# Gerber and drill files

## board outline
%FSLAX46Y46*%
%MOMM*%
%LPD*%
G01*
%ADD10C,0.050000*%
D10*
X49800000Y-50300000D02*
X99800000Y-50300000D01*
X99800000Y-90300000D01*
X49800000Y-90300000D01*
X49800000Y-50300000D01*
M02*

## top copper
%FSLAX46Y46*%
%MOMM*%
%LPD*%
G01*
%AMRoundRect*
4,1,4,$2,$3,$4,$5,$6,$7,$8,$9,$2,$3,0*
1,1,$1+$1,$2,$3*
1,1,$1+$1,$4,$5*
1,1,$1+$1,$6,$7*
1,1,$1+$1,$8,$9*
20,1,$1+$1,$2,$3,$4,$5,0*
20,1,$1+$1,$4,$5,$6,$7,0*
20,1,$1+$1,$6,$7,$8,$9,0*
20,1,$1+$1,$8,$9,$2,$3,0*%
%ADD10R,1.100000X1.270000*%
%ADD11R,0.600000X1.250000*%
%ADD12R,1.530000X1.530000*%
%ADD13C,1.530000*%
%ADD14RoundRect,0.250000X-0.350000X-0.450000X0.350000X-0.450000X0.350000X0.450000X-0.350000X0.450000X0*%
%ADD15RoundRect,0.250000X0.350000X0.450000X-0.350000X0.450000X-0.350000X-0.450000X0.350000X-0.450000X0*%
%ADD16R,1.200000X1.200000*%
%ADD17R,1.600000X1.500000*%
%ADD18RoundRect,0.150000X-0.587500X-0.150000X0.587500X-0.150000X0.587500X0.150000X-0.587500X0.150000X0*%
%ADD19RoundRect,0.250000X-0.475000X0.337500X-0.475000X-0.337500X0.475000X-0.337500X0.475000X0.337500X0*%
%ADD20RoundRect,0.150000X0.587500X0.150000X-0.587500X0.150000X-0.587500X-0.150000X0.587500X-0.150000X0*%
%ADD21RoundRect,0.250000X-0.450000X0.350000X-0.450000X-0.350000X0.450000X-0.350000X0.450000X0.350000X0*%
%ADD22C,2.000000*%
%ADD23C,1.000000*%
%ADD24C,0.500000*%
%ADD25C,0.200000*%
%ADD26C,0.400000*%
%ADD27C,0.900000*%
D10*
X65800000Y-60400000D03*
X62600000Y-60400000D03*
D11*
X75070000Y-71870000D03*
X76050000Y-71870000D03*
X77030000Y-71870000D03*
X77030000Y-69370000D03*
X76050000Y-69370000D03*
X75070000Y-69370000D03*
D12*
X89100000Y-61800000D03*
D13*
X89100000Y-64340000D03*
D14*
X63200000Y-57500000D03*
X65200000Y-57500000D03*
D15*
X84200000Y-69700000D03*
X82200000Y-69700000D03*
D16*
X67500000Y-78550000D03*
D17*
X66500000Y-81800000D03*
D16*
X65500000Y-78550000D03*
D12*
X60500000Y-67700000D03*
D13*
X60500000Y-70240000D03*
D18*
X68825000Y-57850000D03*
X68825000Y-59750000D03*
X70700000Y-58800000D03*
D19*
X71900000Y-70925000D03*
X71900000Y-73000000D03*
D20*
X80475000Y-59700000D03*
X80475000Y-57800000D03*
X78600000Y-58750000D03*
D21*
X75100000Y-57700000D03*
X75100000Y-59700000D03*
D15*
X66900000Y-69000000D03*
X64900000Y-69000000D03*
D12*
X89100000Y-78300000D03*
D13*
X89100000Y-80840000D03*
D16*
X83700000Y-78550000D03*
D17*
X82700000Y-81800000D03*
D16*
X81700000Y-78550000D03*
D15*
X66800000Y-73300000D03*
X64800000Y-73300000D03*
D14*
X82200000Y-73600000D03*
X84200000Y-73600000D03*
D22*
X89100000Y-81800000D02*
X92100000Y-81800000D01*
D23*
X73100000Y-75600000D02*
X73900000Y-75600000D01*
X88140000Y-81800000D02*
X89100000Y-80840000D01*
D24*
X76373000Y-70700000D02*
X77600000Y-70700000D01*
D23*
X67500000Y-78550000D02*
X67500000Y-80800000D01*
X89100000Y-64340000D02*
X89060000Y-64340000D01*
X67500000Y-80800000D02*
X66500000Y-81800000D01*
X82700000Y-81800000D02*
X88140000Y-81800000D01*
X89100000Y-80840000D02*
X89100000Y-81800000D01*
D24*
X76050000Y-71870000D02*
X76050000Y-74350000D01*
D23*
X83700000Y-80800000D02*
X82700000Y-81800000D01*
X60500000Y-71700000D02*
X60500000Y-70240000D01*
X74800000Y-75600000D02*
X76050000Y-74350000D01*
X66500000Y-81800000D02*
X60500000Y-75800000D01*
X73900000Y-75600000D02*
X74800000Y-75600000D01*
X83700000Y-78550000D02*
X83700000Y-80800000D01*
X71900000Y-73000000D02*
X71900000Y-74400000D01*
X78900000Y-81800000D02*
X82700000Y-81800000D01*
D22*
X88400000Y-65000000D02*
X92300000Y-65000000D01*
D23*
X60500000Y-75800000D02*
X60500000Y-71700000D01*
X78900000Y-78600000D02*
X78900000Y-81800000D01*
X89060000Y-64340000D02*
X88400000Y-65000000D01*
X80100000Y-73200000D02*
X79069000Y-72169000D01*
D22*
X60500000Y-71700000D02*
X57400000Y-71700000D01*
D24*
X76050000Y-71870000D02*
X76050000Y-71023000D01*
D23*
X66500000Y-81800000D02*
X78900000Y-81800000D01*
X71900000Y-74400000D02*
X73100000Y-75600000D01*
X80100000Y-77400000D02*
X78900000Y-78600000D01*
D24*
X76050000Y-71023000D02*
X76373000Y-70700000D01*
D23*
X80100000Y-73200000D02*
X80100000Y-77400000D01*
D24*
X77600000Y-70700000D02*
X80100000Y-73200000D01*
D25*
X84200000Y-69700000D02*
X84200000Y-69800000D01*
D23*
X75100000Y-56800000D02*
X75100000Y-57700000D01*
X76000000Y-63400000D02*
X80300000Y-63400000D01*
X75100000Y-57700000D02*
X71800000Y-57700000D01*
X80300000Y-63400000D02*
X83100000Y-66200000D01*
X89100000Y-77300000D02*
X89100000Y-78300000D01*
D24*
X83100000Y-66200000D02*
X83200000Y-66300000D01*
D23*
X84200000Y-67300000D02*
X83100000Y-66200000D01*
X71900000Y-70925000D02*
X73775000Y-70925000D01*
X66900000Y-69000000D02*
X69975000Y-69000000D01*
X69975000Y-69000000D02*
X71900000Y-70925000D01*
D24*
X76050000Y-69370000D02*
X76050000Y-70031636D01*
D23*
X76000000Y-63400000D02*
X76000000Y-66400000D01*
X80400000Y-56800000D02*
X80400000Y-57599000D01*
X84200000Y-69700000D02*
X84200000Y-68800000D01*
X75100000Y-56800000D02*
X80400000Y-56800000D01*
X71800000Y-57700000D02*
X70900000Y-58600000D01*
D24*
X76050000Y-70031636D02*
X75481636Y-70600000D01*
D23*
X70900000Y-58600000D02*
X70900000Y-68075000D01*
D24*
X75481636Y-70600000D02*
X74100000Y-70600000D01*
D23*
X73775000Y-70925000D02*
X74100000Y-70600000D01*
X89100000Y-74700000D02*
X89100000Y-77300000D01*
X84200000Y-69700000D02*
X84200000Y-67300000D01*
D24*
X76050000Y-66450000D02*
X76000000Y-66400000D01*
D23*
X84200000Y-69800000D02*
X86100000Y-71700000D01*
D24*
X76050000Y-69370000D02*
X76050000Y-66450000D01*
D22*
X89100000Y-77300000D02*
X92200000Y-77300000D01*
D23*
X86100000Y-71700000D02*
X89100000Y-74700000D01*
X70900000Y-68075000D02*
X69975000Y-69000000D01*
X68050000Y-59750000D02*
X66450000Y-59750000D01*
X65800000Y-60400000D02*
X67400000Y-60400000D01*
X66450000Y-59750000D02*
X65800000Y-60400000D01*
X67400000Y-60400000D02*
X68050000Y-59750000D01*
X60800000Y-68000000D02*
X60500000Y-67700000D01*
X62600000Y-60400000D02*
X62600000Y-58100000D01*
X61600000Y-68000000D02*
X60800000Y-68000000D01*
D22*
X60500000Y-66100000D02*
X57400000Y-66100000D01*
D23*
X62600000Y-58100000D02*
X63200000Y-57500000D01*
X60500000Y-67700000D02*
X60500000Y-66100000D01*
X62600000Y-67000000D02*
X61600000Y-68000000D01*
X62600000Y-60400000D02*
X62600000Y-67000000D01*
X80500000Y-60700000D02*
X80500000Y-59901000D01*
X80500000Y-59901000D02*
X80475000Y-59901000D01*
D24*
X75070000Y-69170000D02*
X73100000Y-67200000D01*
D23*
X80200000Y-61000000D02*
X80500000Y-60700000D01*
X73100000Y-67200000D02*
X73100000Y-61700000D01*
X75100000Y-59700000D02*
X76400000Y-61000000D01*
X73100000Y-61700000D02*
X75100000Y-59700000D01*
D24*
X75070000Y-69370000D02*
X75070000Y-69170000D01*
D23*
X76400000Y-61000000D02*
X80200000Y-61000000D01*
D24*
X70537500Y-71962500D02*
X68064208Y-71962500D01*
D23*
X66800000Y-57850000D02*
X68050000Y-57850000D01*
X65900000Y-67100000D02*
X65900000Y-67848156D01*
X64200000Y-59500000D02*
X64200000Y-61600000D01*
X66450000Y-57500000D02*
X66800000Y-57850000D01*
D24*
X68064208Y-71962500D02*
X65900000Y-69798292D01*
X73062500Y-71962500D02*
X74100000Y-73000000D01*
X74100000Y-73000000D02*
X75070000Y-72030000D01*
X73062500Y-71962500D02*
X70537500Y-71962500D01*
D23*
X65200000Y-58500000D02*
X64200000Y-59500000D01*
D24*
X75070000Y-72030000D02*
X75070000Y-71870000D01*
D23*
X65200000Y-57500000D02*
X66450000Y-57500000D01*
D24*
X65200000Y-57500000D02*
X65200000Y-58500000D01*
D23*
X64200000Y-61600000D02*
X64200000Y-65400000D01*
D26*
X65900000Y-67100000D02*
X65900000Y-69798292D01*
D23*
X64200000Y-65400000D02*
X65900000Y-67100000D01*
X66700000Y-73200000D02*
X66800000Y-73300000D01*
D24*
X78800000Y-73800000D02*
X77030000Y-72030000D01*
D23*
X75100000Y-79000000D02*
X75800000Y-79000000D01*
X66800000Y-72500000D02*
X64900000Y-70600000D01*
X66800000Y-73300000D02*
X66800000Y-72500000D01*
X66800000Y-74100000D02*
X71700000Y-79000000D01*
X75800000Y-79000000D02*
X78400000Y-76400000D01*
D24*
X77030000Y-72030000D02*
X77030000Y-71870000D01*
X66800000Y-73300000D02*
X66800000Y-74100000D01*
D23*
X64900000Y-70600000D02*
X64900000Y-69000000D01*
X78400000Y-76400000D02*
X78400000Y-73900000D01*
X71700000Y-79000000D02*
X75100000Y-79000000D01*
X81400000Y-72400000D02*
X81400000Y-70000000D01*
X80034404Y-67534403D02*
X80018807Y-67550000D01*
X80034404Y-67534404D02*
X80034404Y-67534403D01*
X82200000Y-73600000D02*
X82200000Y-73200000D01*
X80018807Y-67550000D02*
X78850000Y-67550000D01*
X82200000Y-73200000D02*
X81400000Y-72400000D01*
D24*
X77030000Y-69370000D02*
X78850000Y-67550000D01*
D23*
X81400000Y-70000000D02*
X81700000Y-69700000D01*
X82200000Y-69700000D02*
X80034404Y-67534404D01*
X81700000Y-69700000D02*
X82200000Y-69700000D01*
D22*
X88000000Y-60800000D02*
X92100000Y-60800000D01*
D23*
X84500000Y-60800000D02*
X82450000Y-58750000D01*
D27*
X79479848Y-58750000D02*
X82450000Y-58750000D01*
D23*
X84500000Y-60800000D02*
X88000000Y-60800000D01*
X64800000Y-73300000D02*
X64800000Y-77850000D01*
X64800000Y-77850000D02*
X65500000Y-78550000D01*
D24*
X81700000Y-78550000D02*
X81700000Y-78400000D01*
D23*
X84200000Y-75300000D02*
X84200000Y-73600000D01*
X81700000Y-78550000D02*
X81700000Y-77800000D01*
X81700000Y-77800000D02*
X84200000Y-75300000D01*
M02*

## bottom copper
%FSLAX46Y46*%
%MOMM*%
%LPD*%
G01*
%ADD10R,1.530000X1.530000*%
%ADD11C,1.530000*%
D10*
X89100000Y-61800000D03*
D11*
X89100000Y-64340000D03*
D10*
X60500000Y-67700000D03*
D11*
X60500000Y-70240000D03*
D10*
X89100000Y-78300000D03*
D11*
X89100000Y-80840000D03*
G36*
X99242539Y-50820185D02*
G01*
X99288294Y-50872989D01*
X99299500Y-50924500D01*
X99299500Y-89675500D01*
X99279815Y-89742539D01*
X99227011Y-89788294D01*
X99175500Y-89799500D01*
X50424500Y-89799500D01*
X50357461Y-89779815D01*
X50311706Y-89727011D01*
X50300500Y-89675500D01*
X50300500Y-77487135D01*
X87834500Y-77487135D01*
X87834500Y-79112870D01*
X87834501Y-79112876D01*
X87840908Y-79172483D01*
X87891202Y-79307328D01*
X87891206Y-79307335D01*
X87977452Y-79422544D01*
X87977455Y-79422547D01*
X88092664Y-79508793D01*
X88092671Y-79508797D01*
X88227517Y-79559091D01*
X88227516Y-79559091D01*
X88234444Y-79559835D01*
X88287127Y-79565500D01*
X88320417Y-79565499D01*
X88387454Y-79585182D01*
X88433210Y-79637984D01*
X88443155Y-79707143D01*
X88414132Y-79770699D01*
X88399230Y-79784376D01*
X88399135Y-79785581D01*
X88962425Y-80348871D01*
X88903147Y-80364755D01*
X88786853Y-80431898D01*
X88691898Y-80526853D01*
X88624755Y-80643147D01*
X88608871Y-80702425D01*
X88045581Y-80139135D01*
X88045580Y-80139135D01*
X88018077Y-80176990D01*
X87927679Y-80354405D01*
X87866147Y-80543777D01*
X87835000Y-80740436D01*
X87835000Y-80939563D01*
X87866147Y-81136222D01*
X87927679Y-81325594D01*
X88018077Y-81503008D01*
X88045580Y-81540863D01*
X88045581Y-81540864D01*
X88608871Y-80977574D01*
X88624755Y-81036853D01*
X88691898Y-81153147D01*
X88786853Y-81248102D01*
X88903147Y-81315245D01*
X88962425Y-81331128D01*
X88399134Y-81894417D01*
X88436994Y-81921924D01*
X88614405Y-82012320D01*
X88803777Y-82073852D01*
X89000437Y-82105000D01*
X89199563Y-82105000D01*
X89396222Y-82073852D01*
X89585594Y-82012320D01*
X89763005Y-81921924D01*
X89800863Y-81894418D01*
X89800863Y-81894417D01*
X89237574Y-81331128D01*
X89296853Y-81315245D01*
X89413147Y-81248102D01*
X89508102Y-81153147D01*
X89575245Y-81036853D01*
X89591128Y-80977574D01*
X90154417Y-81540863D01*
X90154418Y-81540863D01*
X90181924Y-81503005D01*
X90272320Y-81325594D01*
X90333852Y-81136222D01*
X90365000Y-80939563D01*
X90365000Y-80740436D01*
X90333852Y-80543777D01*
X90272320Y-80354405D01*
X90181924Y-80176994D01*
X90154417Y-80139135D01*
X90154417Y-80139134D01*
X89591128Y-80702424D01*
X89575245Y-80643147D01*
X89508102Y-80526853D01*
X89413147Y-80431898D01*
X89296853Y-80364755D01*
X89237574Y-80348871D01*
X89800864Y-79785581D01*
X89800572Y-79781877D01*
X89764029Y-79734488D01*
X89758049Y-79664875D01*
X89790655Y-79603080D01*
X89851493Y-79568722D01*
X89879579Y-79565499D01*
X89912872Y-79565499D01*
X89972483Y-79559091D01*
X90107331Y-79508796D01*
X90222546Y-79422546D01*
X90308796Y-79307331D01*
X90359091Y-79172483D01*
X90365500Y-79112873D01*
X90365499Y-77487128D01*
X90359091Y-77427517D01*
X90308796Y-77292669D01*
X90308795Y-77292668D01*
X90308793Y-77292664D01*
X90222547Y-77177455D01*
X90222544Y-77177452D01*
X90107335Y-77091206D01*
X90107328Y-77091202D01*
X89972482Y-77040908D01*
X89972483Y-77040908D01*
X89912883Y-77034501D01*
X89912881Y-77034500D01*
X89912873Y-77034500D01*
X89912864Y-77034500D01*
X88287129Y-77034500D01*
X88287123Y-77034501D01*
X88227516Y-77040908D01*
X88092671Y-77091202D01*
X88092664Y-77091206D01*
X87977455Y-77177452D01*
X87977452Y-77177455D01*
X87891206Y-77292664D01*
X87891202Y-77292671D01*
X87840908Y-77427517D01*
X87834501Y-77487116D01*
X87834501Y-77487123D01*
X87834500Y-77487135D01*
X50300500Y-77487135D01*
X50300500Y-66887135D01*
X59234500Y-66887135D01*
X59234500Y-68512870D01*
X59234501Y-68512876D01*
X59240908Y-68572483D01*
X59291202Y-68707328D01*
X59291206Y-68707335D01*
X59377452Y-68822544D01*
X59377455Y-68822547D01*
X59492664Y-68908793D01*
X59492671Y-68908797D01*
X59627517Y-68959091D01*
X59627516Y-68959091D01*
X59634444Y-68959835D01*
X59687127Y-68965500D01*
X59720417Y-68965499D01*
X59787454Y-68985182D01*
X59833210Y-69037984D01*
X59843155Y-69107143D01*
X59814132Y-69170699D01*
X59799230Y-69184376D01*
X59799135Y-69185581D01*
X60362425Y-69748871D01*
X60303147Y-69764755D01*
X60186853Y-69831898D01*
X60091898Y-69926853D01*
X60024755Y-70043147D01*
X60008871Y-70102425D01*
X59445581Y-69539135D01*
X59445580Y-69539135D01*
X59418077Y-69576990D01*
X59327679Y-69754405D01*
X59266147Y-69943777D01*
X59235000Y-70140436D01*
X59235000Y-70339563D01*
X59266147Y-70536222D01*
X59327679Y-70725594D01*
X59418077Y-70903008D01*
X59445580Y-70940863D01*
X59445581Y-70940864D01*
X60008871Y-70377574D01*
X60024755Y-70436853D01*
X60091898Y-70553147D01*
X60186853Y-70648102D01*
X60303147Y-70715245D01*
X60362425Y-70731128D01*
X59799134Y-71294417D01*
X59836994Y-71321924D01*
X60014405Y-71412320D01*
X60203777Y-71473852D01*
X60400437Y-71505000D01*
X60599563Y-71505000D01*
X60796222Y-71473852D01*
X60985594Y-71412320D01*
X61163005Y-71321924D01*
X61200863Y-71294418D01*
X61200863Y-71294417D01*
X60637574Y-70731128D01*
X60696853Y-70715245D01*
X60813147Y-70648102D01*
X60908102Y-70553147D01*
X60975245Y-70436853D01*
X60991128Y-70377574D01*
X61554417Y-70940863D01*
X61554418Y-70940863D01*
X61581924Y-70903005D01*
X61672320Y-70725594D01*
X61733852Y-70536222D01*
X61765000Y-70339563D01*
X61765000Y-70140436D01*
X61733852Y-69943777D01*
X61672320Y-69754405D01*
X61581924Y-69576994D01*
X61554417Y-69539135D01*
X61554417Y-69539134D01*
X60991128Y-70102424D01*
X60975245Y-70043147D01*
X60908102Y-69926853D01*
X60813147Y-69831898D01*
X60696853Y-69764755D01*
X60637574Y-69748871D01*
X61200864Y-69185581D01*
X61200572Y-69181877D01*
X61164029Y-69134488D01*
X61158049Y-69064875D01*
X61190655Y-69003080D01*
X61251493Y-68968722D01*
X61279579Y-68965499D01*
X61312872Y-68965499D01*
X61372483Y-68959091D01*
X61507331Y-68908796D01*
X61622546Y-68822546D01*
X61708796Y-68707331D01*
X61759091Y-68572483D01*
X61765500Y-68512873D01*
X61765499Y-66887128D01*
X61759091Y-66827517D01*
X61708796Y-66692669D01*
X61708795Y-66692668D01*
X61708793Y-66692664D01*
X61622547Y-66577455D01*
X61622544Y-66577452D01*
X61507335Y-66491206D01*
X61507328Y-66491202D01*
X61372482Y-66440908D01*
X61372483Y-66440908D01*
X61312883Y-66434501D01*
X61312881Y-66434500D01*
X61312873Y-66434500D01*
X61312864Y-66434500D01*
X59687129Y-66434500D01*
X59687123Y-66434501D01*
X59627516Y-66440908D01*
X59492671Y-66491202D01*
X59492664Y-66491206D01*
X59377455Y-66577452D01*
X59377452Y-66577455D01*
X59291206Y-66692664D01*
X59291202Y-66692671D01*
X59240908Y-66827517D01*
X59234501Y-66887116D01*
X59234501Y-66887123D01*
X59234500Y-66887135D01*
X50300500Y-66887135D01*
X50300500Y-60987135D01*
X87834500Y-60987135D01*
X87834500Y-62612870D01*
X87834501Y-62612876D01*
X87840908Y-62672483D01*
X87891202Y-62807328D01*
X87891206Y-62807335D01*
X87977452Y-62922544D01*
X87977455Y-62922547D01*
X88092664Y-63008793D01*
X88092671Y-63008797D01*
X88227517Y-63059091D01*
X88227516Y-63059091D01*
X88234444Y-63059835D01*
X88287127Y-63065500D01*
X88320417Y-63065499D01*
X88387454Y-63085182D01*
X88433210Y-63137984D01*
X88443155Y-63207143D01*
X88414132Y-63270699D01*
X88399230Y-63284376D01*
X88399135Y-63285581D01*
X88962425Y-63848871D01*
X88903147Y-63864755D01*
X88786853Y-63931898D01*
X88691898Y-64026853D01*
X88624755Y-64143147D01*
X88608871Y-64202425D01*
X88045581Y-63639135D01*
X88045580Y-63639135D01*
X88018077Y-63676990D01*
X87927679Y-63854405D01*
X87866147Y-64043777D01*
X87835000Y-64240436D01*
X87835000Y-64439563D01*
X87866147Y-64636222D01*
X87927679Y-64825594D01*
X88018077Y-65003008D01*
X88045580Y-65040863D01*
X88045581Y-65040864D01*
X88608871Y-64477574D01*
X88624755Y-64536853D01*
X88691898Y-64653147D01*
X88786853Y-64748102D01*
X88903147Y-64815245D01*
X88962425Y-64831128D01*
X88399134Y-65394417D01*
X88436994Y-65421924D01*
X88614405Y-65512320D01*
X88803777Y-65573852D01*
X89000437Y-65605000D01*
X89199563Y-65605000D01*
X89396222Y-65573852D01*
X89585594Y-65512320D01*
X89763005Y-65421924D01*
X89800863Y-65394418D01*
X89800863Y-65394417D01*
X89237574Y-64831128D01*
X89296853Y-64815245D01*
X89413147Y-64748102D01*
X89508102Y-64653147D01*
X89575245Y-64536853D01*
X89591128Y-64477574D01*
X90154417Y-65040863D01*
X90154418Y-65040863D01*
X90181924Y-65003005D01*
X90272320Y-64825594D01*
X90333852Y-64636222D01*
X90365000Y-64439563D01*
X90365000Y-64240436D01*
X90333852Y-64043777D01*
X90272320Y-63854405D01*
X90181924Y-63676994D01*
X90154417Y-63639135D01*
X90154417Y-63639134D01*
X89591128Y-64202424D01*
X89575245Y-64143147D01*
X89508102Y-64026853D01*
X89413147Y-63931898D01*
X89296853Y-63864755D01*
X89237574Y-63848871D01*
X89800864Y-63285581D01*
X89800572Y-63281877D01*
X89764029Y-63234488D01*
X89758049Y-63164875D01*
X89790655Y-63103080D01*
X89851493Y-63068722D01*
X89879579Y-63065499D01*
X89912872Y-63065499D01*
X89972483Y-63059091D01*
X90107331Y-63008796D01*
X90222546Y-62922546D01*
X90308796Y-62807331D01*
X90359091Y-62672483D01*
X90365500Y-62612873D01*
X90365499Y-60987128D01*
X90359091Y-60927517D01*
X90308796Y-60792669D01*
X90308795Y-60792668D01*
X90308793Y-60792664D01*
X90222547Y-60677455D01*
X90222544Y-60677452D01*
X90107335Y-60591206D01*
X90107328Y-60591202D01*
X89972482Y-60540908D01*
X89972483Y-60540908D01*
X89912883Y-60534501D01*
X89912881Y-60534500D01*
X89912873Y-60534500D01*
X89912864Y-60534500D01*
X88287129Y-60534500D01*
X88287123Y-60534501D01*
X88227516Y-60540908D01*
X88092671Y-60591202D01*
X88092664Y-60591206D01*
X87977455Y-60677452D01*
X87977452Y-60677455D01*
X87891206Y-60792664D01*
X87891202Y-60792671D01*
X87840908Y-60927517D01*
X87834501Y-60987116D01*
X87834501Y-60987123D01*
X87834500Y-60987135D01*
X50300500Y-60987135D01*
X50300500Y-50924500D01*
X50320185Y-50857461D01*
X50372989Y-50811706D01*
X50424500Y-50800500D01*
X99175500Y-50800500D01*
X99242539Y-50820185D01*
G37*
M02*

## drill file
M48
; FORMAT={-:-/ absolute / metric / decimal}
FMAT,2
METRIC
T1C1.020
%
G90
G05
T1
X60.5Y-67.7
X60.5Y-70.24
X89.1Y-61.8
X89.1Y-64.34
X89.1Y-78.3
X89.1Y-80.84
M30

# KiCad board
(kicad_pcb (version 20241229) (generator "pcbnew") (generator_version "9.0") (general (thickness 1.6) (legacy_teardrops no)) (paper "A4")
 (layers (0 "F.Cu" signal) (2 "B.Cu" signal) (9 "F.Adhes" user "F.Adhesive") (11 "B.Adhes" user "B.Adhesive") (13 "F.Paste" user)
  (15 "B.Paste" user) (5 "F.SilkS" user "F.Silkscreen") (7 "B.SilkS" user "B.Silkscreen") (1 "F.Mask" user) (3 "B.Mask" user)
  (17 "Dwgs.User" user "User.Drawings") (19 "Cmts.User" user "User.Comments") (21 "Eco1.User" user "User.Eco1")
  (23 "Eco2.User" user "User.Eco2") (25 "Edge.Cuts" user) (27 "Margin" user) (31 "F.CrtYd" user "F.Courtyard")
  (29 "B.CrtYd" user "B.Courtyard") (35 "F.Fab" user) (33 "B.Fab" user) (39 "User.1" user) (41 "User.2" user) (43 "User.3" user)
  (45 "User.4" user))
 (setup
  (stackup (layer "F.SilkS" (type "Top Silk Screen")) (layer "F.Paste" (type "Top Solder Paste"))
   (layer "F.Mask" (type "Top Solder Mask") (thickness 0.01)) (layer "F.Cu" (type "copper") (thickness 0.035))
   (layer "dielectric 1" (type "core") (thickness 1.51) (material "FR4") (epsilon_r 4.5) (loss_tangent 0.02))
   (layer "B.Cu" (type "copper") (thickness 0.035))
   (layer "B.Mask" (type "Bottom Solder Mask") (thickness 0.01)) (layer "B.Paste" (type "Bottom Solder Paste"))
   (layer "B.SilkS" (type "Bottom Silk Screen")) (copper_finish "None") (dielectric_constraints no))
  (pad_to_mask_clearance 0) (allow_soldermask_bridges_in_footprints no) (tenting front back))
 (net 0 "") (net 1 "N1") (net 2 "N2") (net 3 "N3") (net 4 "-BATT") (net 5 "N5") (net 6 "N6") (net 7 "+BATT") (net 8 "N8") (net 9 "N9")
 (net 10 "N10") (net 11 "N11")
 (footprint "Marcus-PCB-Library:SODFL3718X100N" (layer "F.Cu") (at 64.2 60.4 180)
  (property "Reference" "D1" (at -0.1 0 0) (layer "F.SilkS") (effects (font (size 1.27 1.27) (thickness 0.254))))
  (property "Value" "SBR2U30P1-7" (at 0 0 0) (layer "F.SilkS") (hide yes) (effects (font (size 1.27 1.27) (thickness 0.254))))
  (pad "1" smd rect (at -1.6 0 180) (size 1.1 1.27) (layers "F.Cu" "F.Mask" "F.Paste") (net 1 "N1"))
  (pad "2" smd rect (at 1.6 0 180) (size 1.1 1.27) (layers "F.Cu" "F.Mask" "F.Paste") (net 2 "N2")))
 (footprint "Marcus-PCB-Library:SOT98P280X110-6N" (layer "F.Cu") (at 76.05 70.62 90)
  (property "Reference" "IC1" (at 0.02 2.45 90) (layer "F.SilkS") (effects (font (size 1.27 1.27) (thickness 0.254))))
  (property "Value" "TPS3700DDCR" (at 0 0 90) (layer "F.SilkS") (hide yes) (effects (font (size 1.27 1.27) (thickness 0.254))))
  (pad "1" smd rect (at -1.25 -0.98 180) (size 0.6 1.25) (layers "F.Cu" "F.Mask" "F.Paste") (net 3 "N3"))
  (pad "2" smd rect (at -1.25 0 180) (size 0.6 1.25) (layers "F.Cu" "F.Mask" "F.Paste") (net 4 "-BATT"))
  (pad "3" smd rect (at -1.25 0.98 180) (size 0.6 1.25) (layers "F.Cu" "F.Mask" "F.Paste") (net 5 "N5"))
  (pad "4" smd rect (at 1.25 0.98 180) (size 0.6 1.25) (layers "F.Cu" "F.Mask" "F.Paste") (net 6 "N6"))
  (pad "5" smd rect (at 1.25 0 180) (size 0.6 1.25) (layers "F.Cu" "F.Mask" "F.Paste") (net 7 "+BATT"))
  (pad "6" smd rect (at 1.25 -0.98 180) (size 0.6 1.25) (layers "F.Cu" "F.Mask" "F.Paste") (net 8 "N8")))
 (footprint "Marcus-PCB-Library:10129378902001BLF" (layer "F.Cu") (at 89.1 61.8 -90)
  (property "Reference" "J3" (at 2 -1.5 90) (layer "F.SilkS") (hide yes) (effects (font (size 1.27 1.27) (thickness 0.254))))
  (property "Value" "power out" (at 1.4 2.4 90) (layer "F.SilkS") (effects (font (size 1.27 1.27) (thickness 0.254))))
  (pad "1" thru_hole rect (at 0 0 270) (size 1.53 1.53) (drill 1.02) (layers "*.Cu" "*.Mask") (remove_unused_layers no) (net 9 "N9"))
  (pad "2" thru_hole circle (at 2.54 0 270) (size 1.53 1.53) (drill 1.02) (layers "*.Cu" "*.Mask") (remove_unused_layers no) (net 4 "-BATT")))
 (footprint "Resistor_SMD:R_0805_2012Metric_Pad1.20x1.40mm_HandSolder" (layer "F.Cu") (at 64.2 57.5)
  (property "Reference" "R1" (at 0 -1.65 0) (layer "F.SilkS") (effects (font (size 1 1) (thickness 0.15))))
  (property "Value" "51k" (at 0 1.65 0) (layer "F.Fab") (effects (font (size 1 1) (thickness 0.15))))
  (pad "1" smd roundrect (at -1 0) (size 1.2 1.4) (layers "F.Cu" "F.Mask" "F.Paste") (roundrect_rratio 0.208333) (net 2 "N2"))
  (pad "2" smd roundrect (at 1 0) (size 1.2 1.4) (layers "F.Cu" "F.Mask" "F.Paste") (roundrect_rratio 0.208333) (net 3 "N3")))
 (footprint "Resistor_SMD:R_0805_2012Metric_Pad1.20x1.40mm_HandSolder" (layer "F.Cu") (at 83.2 69.7 180)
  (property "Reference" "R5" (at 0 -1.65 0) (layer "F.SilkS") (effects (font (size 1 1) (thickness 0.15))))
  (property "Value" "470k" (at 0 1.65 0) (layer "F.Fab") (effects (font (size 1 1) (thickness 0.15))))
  (pad "1" smd roundrect (at -1 0 180) (size 1.2 1.4) (layers "F.Cu" "F.Mask" "F.Paste") (roundrect_rratio 0.208333) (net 7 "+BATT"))
  (pad "2" smd roundrect (at 1 0 180) (size 1.2 1.4) (layers "F.Cu" "F.Mask" "F.Paste") (roundrect_rratio 0.208333) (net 6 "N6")))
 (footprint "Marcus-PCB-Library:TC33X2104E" (layer "F.Cu") (at 66.5 80.35 180)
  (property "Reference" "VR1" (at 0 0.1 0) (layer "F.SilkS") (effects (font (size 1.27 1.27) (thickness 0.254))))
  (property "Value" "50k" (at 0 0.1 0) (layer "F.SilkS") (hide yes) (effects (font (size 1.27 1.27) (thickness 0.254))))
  (pad "1" smd rect (at -1 1.8 270) (size 1.2 1.2) (layers "F.Cu" "F.Mask" "F.Paste") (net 4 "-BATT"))
  (pad "2" smd rect (at 0 -1.45 270) (size 1.5 1.6) (layers "F.Cu" "F.Mask" "F.Paste") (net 4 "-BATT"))
  (pad "3" smd rect (at 1 1.8 270) (size 1.2 1.2) (layers "F.Cu" "F.Mask" "F.Paste") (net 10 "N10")))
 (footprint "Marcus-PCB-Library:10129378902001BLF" (layer "F.Cu") (at 60.5 67.7 -90)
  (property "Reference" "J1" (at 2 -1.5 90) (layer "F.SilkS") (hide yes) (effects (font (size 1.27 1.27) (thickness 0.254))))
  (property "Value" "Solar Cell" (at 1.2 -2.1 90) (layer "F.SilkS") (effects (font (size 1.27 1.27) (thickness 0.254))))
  (pad "1" thru_hole rect (at 0 0 270) (size 1.53 1.53) (drill 1.02) (layers "*.Cu" "*.Mask") (remove_unused_layers no) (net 2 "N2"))
  (pad "2" thru_hole circle (at 2.54 0 270) (size 1.53 1.53) (drill 1.02) (layers "*.Cu" "*.Mask") (remove_unused_layers no) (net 4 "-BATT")))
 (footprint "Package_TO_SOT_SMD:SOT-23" (layer "F.Cu") (at 69.7625 58.8)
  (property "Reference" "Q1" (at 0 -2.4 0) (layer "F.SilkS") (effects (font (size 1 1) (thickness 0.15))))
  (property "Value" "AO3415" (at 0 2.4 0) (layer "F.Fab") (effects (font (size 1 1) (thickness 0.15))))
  (pad "1" smd roundrect (at -0.9375 -0.95) (size 1.475 0.6) (layers "F.Cu" "F.Mask" "F.Paste") (roundrect_rratio 0.25) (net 3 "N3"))
  (pad "2" smd roundrect (at -0.9375 0.95) (size 1.475 0.6) (layers "F.Cu" "F.Mask" "F.Paste") (roundrect_rratio 0.25) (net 1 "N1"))
  (pad "3" smd roundrect (at 0.9375 0) (size 1.475 0.6) (layers "F.Cu" "F.Mask" "F.Paste") (roundrect_rratio 0.25) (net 7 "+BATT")))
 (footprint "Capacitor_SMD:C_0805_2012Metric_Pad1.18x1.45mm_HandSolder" (layer "F.Cu") (at 71.9 71.9625 -90)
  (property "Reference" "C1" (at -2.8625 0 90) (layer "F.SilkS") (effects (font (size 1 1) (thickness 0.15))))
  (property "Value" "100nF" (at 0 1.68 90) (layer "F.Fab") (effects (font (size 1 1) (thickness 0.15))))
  (pad "1" smd roundrect (at -1.0375 0 270) (size 1.175 1.45) (layers "F.Cu" "F.Mask" "F.Paste") (roundrect_rratio 0.212766) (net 7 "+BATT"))
  (pad "2" smd roundrect (at 1.0375 0 270) (size 1.175 1.45) (layers "F.Cu" "F.Mask" "F.Paste") (roundrect_rratio 0.212766) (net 4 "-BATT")))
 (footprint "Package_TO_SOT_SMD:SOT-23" (layer "F.Cu") (at 79.5375 58.75 180)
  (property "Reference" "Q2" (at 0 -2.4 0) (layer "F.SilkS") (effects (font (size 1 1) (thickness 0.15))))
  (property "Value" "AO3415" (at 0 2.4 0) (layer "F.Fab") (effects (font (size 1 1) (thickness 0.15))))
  (pad "1" smd roundrect (at -0.9375 -0.95 180) (size 1.475 0.6) (layers "F.Cu" "F.Mask" "F.Paste") (roundrect_rratio 0.25) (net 8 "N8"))
  (pad "2" smd roundrect (at -0.9375 0.95 180) (size 1.475 0.6) (layers "F.Cu" "F.Mask" "F.Paste") (roundrect_rratio 0.25) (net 7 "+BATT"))
  (pad "3" smd roundrect (at 0.9375 0 180) (size 1.475 0.6) (layers "F.Cu" "F.Mask" "F.Paste") (roundrect_rratio 0.25) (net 9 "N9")))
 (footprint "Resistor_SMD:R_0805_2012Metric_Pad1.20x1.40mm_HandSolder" (layer "F.Cu") (at 75.1 58.7 -90)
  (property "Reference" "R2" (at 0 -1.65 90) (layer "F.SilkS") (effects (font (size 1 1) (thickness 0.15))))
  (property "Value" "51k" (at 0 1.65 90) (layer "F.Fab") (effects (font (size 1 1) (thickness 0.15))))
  (pad "1" smd roundrect (at -1 0 270) (size 1.2 1.4) (layers "F.Cu" "F.Mask" "F.Paste") (roundrect_rratio 0.208333) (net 7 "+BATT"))
  (pad "2" smd roundrect (at 1 0 270) (size 1.2 1.4) (layers "F.Cu" "F.Mask" "F.Paste") (roundrect_rratio 0.208333) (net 8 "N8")))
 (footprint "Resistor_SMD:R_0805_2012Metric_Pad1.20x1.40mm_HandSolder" (layer "F.Cu") (at 65.9 69 180)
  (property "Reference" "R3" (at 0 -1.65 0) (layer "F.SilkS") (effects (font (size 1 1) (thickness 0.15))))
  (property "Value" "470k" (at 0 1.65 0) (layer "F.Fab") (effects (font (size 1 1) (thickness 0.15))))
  (pad "1" smd roundrect (at -1 0 180) (size 1.2 1.4) (layers "F.Cu" "F.Mask" "F.Paste") (roundrect_rratio 0.208333) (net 7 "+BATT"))
  (pad "2" smd roundrect (at 1 0 180) (size 1.2 1.4) (layers "F.Cu" "F.Mask" "F.Paste") (roundrect_rratio 0.208333) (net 5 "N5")))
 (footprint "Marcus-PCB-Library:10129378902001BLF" (layer "F.Cu") (at 89.1 78.3 -90)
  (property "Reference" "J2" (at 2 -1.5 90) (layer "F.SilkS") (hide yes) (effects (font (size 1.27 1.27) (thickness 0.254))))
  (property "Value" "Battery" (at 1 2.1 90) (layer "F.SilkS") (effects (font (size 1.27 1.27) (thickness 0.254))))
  (pad "1" thru_hole rect (at 0 0 270) (size 1.53 1.53) (drill 1.02) (layers "*.Cu" "*.Mask") (remove_unused_layers no) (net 7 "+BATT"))
  (pad "2" thru_hole circle (at 2.54 0 270) (size 1.53 1.53) (drill 1.02) (layers "*.Cu" "*.Mask") (remove_unused_layers no) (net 4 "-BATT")))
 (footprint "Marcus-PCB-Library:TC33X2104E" (layer "F.Cu") (at 82.7 80.35 180)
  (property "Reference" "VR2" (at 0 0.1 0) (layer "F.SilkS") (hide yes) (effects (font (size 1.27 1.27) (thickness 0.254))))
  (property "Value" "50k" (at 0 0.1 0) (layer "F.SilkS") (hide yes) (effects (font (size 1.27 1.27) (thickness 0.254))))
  (pad "1" smd rect (at -1 1.8 270) (size 1.2 1.2) (layers "F.Cu" "F.Mask" "F.Paste") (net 4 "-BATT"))
  (pad "2" smd rect (at 0 -1.45 270) (size 1.5 1.6) (layers "F.Cu" "F.Mask" "F.Paste") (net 4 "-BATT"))
  (pad "3" smd rect (at 1 1.8 270) (size 1.2 1.2) (layers "F.Cu" "F.Mask" "F.Paste") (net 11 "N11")))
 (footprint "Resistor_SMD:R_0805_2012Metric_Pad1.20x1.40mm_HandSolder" (layer "F.Cu") (at 65.8 73.3 180)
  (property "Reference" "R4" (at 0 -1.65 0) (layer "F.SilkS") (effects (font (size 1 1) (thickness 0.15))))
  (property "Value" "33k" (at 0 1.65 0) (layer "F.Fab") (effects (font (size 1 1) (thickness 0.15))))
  (pad "1" smd roundrect (at -1 0 180) (size 1.2 1.4) (layers "F.Cu" "F.Mask" "F.Paste") (roundrect_rratio 0.208333) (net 5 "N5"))
  (pad "2" smd roundrect (at 1 0 180) (size 1.2 1.4) (layers "F.Cu" "F.Mask" "F.Paste") (roundrect_rratio 0.208333) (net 10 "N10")))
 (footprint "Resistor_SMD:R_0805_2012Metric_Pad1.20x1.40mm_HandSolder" (layer "F.Cu") (at 83.2 73.6)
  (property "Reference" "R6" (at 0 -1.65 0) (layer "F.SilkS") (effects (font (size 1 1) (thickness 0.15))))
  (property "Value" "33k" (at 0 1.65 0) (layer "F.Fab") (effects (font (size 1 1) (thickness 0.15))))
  (pad "1" smd roundrect (at -1 0) (size 1.2 1.4) (layers "F.Cu" "F.Mask" "F.Paste") (roundrect_rratio 0.208333) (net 6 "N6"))
  (pad "2" smd roundrect (at 1 0) (size 1.2 1.4) (layers "F.Cu" "F.Mask" "F.Paste") (roundrect_rratio 0.208333) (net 11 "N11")))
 (gr_rect (start 49.8 50.3) (end 99.8 90.3) (stroke (width 0.05) (type default)) (fill no) (layer "Edge.Cuts"))
 (segment (start 89.1 81.8) (end 92.1 81.8) (width 2) (layer "F.Cu") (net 4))
 (segment (start 73.1 75.6) (end 73.9 75.6) (width 1) (layer "F.Cu") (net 4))
 (segment (start 88.14 81.8) (end 89.1 80.84) (width 1) (layer "F.Cu") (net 4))
 (segment (start 76.373 70.7) (end 77.6 70.7) (width 0.5) (layer "F.Cu") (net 4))
 (segment (start 67.5 78.55) (end 67.5 80.8) (width 1) (layer "F.Cu") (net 4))
 (segment (start 89.1 64.34) (end 89.06 64.34) (width 1) (layer "F.Cu") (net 4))
 (segment (start 67.5 80.8) (end 66.5 81.8) (width 1) (layer "F.Cu") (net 4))
 (segment (start 82.7 81.8) (end 88.14 81.8) (width 1) (layer "F.Cu") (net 4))
 (segment (start 89.1 80.84) (end 89.1 81.8) (width 1) (layer "F.Cu") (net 4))
 (segment (start 76.05 71.87) (end 76.05 74.35) (width 0.5) (layer "F.Cu") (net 4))
 (segment (start 83.7 80.8) (end 82.7 81.8) (width 1) (layer "F.Cu") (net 4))
 (segment (start 60.5 71.7) (end 60.5 70.24) (width 1) (layer "F.Cu") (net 4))
 (segment (start 74.8 75.6) (end 76.05 74.35) (width 1) (layer "F.Cu") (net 4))
 (segment (start 66.5 81.8) (end 60.5 75.8) (width 1) (layer "F.Cu") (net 4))
 (segment (start 73.9 75.6) (end 74.8 75.6) (width 1) (layer "F.Cu") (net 4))
 (segment (start 83.7 78.55) (end 83.7 80.8) (width 1) (layer "F.Cu") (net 4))
 (segment (start 71.9 73) (end 71.9 74.4) (width 1) (layer "F.Cu") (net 4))
 (segment (start 78.9 81.8) (end 82.7 81.8) (width 1) (layer "F.Cu") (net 4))
 (segment (start 88.4 65) (end 92.3 65) (width 2) (layer "F.Cu") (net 4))
 (segment (start 60.5 75.8) (end 60.5 71.7) (width 1) (layer "F.Cu") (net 4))
 (segment (start 78.9 78.6) (end 78.9 81.8) (width 1) (layer "F.Cu") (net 4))
 (segment (start 89.06 64.34) (end 88.4 65) (width 1) (layer "F.Cu") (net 4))
 (segment (start 80.1 73.2) (end 79.069 72.169) (width 1) (layer "F.Cu") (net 4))
 (segment (start 60.5 71.7) (end 57.4 71.7) (width 2) (layer "F.Cu") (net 4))
 (segment (start 76.05 71.87) (end 76.05 71.023) (width 0.5) (layer "F.Cu") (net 4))
 (segment (start 66.5 81.8) (end 78.9 81.8) (width 1) (layer "F.Cu") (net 4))
 (segment (start 71.9 74.4) (end 73.1 75.6) (width 1) (layer "F.Cu") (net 4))
 (segment (start 80.1 77.4) (end 78.9 78.6) (width 1) (layer "F.Cu") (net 4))
 (segment (start 76.05 71.023) (end 76.373 70.7) (width 0.5) (layer "F.Cu") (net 4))
 (segment (start 80.1 73.2) (end 80.1 77.4) (width 1) (layer "F.Cu") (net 4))
 (segment (start 77.6 70.7) (end 80.1 73.2) (width 0.5) (layer "F.Cu") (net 4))
 (segment (start 84.2 69.7) (end 84.2 69.8) (width 0.2) (layer "F.Cu") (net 7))
 (segment (start 75.1 56.8) (end 75.1 57.7) (width 1) (layer "F.Cu") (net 7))
 (segment (start 76 63.4) (end 80.3 63.4) (width 1) (layer "F.Cu") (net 7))
 (segment (start 75.1 57.7) (end 71.8 57.7) (width 1) (layer "F.Cu") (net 7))
 (segment (start 80.3 63.4) (end 83.1 66.2) (width 1) (layer "F.Cu") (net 7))
 (segment (start 89.1 77.3) (end 89.1 78.3) (width 1) (layer "F.Cu") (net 7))
 (segment (start 83.1 66.2) (end 83.2 66.3) (width 0.5) (layer "F.Cu") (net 7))
 (segment (start 84.2 67.3) (end 83.1 66.2) (width 1) (layer "F.Cu") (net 7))
 (segment (start 71.9 70.925) (end 73.775 70.925) (width 1) (layer "F.Cu") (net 7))
 (segment (start 66.9 69) (end 69.975 69) (width 1) (layer "F.Cu") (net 7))
 (segment (start 69.975 69) (end 71.9 70.925) (width 1) (layer "F.Cu") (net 7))
 (segment (start 76.05 69.37) (end 76.05 70.031636) (width 0.5) (layer "F.Cu") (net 7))
 (segment (start 76 63.4) (end 76 66.4) (width 1) (layer "F.Cu") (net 7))
 (segment (start 80.4 56.8) (end 80.4 57.599) (width 1) (layer "F.Cu") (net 7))
 (segment (start 84.2 69.7) (end 84.2 68.8) (width 1) (layer "F.Cu") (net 7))
 (segment (start 75.1 56.8) (end 80.4 56.8) (width 1) (layer "F.Cu") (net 7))
 (segment (start 71.8 57.7) (end 70.9 58.6) (width 1) (layer "F.Cu") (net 7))
 (segment (start 76.05 70.031636) (end 75.481636 70.6) (width 0.5) (layer "F.Cu") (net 7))
 (segment (start 70.9 58.6) (end 70.9 68.075) (width 1) (layer "F.Cu") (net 7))
 (segment (start 75.481636 70.6) (end 74.1 70.6) (width 0.5) (layer "F.Cu") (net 7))
 (segment (start 73.775 70.925) (end 74.1 70.6) (width 1) (layer "F.Cu") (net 7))
 (segment (start 89.1 74.7) (end 89.1 77.3) (width 1) (layer "F.Cu") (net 7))
 (segment (start 84.2 69.7) (end 84.2 67.3) (width 1) (layer "F.Cu") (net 7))
 (segment (start 76.05 66.45) (end 76 66.4) (width 0.5) (layer "F.Cu") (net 7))
 (segment (start 84.2 69.8) (end 86.1 71.7) (width 1) (layer "F.Cu") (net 7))
 (segment (start 76.05 69.37) (end 76.05 66.45) (width 0.5) (layer "F.Cu") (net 7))
 (segment (start 89.1 77.3) (end 92.2 77.3) (width 2) (layer "F.Cu") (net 7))
 (segment (start 86.1 71.7) (end 89.1 74.7) (width 1) (layer "F.Cu") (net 7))
 (segment (start 70.9 68.075) (end 69.975 69) (width 1) (layer "F.Cu") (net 7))
 (segment (start 68.05 59.75) (end 66.45 59.75) (width 1) (layer "F.Cu") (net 1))
 (segment (start 65.8 60.4) (end 67.4 60.4) (width 1) (layer "F.Cu") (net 1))
 (segment (start 66.45 59.75) (end 65.8 60.4) (width 1) (layer "F.Cu") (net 1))
 (segment (start 67.4 60.4) (end 68.05 59.75) (width 1) (layer "F.Cu") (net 1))
 (segment (start 60.8 68) (end 60.5 67.7) (width 1) (layer "F.Cu") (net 2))
 (segment (start 62.6 60.4) (end 62.6 58.1) (width 1) (layer "F.Cu") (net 2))
 (segment (start 61.6 68) (end 60.8 68) (width 1) (layer "F.Cu") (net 2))
 (segment (start 60.5 66.1) (end 57.4 66.1) (width 2) (layer "F.Cu") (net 2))
 (segment (start 62.6 58.1) (end 63.2 57.5) (width 1) (layer "F.Cu") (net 2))
 (segment (start 60.5 67.7) (end 60.5 66.1) (width 1) (layer "F.Cu") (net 2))
 (segment (start 62.6 67) (end 61.6 68) (width 1) (layer "F.Cu") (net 2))
 (segment (start 62.6 60.4) (end 62.6 67) (width 1) (layer "F.Cu") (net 2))
 (segment (start 80.5 60.7) (end 80.5 59.901) (width 1) (layer "F.Cu") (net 8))
 (segment (start 80.5 59.901) (end 80.475 59.901) (width 1) (layer "F.Cu") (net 8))
 (segment (start 75.07 69.17) (end 73.1 67.2) (width 0.5) (layer "F.Cu") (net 8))
 (segment (start 80.2 61) (end 80.5 60.7) (width 1) (layer "F.Cu") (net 8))
 (segment (start 73.1 67.2) (end 73.1 61.7) (width 1) (layer "F.Cu") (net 8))
 (segment (start 75.1 59.7) (end 76.4 61) (width 1) (layer "F.Cu") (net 8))
 (segment (start 73.1 61.7) (end 75.1 59.7) (width 1) (layer "F.Cu") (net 8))
 (segment (start 75.07 69.37) (end 75.07 69.17) (width 0.5) (layer "F.Cu") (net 8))
 (segment (start 76.4 61) (end 80.2 61) (width 1) (layer "F.Cu") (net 8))
 (segment (start 70.5375 71.9625) (end 68.064208 71.9625) (width 0.5) (layer "F.Cu") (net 3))
 (segment (start 66.8 57.85) (end 68.05 57.85) (width 1) (layer "F.Cu") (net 3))
 (segment (start 65.9 67.1) (end 65.9 67.848156) (width 1) (layer "F.Cu") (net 3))
 (segment (start 64.2 59.5) (end 64.2 61.6) (width 1) (layer "F.Cu") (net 3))
 (segment (start 66.45 57.5) (end 66.8 57.85) (width 1) (layer "F.Cu") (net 3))
 (segment (start 68.064208 71.9625) (end 65.9 69.798292) (width 0.5) (layer "F.Cu") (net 3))
 (segment (start 73.0625 71.9625) (end 74.1 73) (width 0.5) (layer "F.Cu") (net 3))
 (segment (start 74.1 73) (end 75.07 72.03) (width 0.5) (layer "F.Cu") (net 3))
 (segment (start 73.0625 71.9625) (end 70.5375 71.9625) (width 0.5) (layer "F.Cu") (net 3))
 (segment (start 65.2 58.5) (end 64.2 59.5) (width 1) (layer "F.Cu") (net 3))
 (segment (start 75.07 72.03) (end 75.07 71.87) (width 0.5) (layer "F.Cu") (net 3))
 (segment (start 65.2 57.5) (end 66.45 57.5) (width 1) (layer "F.Cu") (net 3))
 (segment (start 65.2 57.5) (end 65.2 58.5) (width 0.5) (layer "F.Cu") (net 3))
 (segment (start 64.2 61.6) (end 64.2 65.4) (width 1) (layer "F.Cu") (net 3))
 (segment (start 65.9 67.1) (end 65.9 69.798292) (width 0.4) (layer "F.Cu") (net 3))
 (segment (start 64.2 65.4) (end 65.9 67.1) (width 1) (layer "F.Cu") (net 3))
 (segment (start 66.7 73.2) (end 66.8 73.3) (width 1) (layer "F.Cu") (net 5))
 (segment (start 78.8 73.8) (end 77.03 72.03) (width 0.5) (layer "F.Cu") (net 5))
 (segment (start 75.1 79) (end 75.8 79) (width 1) (layer "F.Cu") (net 5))
 (segment (start 66.8 72.5) (end 64.9 70.6) (width 1) (layer "F.Cu") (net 5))
 (segment (start 66.8 73.3) (end 66.8 72.5) (width 1) (layer "F.Cu") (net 5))
 (segment (start 66.8 74.1) (end 71.7 79) (width 1) (layer "F.Cu") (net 5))
 (segment (start 75.8 79) (end 78.4 76.4) (width 1) (layer "F.Cu") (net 5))
 (segment (start 77.03 72.03) (end 77.03 71.87) (width 0.5) (layer "F.Cu") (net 5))
 (segment (start 66.8 73.3) (end 66.8 74.1) (width 0.5) (layer "F.Cu") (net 5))
 (segment (start 64.9 70.6) (end 64.9 69) (width 1) (layer "F.Cu") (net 5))
 (segment (start 78.4 76.4) (end 78.4 73.9) (width 1) (layer "F.Cu") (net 5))
 (segment (start 71.7 79) (end 75.1 79) (width 1) (layer "F.Cu") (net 5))
 (segment (start 81.4 72.4) (end 81.4 70) (width 1) (layer "F.Cu") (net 6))
 (segment (start 80.034404 67.534403) (end 80.018807 67.55) (width 1) (layer "F.Cu") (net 6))
 (segment (start 80.034404 67.534404) (end 80.034404 67.534403) (width 1) (layer "F.Cu") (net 6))
 (segment (start 82.2 73.6) (end 82.2 73.2) (width 1) (layer "F.Cu") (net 6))
 (segment (start 80.018807 67.55) (end 78.85 67.55) (width 1) (layer "F.Cu") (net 6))
 (segment (start 82.2 73.2) (end 81.4 72.4) (width 1) (layer "F.Cu") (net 6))
 (segment (start 77.03 69.37) (end 78.85 67.55) (width 0.5) (layer "F.Cu") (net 6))
 (segment (start 81.4 70) (end 81.7 69.7) (width 1) (layer "F.Cu") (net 6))
 (segment (start 82.2 69.7) (end 80.034404 67.534404) (width 1) (layer "F.Cu") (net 6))
 (segment (start 81.7 69.7) (end 82.2 69.7) (width 1) (layer "F.Cu") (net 6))
 (segment (start 88 60.8) (end 92.1 60.8) (width 2) (layer "F.Cu") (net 9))
 (segment (start 84.5 60.8) (end 82.45 58.75) (width 1) (layer "F.Cu") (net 9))
 (segment (start 79.479848 58.75) (end 82.45 58.75) (width 0.9) (layer "F.Cu") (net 9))
 (segment (start 84.5 60.8) (end 88 60.8) (width 1) (layer "F.Cu") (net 9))
 (segment (start 64.8 73.3) (end 64.8 77.85) (width 1) (layer "F.Cu") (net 10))
 (segment (start 64.8 77.85) (end 65.5 78.55) (width 1) (layer "F.Cu") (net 10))
 (segment (start 81.7 78.55) (end 81.7 78.4) (width 0.5) (layer "F.Cu") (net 11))
 (segment (start 84.2 75.3) (end 84.2 73.6) (width 1) (layer "F.Cu") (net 11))
 (segment (start 81.7 78.55) (end 81.7 77.8) (width 1) (layer "F.Cu") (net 11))
 (segment (start 81.7 77.8) (end 84.2 75.3) (width 1) (layer "F.Cu") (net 11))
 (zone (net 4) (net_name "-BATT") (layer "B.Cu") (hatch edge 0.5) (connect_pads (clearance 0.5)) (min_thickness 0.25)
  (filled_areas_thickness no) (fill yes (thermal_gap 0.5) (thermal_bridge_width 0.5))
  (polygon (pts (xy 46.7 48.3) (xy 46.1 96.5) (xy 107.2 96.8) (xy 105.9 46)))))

